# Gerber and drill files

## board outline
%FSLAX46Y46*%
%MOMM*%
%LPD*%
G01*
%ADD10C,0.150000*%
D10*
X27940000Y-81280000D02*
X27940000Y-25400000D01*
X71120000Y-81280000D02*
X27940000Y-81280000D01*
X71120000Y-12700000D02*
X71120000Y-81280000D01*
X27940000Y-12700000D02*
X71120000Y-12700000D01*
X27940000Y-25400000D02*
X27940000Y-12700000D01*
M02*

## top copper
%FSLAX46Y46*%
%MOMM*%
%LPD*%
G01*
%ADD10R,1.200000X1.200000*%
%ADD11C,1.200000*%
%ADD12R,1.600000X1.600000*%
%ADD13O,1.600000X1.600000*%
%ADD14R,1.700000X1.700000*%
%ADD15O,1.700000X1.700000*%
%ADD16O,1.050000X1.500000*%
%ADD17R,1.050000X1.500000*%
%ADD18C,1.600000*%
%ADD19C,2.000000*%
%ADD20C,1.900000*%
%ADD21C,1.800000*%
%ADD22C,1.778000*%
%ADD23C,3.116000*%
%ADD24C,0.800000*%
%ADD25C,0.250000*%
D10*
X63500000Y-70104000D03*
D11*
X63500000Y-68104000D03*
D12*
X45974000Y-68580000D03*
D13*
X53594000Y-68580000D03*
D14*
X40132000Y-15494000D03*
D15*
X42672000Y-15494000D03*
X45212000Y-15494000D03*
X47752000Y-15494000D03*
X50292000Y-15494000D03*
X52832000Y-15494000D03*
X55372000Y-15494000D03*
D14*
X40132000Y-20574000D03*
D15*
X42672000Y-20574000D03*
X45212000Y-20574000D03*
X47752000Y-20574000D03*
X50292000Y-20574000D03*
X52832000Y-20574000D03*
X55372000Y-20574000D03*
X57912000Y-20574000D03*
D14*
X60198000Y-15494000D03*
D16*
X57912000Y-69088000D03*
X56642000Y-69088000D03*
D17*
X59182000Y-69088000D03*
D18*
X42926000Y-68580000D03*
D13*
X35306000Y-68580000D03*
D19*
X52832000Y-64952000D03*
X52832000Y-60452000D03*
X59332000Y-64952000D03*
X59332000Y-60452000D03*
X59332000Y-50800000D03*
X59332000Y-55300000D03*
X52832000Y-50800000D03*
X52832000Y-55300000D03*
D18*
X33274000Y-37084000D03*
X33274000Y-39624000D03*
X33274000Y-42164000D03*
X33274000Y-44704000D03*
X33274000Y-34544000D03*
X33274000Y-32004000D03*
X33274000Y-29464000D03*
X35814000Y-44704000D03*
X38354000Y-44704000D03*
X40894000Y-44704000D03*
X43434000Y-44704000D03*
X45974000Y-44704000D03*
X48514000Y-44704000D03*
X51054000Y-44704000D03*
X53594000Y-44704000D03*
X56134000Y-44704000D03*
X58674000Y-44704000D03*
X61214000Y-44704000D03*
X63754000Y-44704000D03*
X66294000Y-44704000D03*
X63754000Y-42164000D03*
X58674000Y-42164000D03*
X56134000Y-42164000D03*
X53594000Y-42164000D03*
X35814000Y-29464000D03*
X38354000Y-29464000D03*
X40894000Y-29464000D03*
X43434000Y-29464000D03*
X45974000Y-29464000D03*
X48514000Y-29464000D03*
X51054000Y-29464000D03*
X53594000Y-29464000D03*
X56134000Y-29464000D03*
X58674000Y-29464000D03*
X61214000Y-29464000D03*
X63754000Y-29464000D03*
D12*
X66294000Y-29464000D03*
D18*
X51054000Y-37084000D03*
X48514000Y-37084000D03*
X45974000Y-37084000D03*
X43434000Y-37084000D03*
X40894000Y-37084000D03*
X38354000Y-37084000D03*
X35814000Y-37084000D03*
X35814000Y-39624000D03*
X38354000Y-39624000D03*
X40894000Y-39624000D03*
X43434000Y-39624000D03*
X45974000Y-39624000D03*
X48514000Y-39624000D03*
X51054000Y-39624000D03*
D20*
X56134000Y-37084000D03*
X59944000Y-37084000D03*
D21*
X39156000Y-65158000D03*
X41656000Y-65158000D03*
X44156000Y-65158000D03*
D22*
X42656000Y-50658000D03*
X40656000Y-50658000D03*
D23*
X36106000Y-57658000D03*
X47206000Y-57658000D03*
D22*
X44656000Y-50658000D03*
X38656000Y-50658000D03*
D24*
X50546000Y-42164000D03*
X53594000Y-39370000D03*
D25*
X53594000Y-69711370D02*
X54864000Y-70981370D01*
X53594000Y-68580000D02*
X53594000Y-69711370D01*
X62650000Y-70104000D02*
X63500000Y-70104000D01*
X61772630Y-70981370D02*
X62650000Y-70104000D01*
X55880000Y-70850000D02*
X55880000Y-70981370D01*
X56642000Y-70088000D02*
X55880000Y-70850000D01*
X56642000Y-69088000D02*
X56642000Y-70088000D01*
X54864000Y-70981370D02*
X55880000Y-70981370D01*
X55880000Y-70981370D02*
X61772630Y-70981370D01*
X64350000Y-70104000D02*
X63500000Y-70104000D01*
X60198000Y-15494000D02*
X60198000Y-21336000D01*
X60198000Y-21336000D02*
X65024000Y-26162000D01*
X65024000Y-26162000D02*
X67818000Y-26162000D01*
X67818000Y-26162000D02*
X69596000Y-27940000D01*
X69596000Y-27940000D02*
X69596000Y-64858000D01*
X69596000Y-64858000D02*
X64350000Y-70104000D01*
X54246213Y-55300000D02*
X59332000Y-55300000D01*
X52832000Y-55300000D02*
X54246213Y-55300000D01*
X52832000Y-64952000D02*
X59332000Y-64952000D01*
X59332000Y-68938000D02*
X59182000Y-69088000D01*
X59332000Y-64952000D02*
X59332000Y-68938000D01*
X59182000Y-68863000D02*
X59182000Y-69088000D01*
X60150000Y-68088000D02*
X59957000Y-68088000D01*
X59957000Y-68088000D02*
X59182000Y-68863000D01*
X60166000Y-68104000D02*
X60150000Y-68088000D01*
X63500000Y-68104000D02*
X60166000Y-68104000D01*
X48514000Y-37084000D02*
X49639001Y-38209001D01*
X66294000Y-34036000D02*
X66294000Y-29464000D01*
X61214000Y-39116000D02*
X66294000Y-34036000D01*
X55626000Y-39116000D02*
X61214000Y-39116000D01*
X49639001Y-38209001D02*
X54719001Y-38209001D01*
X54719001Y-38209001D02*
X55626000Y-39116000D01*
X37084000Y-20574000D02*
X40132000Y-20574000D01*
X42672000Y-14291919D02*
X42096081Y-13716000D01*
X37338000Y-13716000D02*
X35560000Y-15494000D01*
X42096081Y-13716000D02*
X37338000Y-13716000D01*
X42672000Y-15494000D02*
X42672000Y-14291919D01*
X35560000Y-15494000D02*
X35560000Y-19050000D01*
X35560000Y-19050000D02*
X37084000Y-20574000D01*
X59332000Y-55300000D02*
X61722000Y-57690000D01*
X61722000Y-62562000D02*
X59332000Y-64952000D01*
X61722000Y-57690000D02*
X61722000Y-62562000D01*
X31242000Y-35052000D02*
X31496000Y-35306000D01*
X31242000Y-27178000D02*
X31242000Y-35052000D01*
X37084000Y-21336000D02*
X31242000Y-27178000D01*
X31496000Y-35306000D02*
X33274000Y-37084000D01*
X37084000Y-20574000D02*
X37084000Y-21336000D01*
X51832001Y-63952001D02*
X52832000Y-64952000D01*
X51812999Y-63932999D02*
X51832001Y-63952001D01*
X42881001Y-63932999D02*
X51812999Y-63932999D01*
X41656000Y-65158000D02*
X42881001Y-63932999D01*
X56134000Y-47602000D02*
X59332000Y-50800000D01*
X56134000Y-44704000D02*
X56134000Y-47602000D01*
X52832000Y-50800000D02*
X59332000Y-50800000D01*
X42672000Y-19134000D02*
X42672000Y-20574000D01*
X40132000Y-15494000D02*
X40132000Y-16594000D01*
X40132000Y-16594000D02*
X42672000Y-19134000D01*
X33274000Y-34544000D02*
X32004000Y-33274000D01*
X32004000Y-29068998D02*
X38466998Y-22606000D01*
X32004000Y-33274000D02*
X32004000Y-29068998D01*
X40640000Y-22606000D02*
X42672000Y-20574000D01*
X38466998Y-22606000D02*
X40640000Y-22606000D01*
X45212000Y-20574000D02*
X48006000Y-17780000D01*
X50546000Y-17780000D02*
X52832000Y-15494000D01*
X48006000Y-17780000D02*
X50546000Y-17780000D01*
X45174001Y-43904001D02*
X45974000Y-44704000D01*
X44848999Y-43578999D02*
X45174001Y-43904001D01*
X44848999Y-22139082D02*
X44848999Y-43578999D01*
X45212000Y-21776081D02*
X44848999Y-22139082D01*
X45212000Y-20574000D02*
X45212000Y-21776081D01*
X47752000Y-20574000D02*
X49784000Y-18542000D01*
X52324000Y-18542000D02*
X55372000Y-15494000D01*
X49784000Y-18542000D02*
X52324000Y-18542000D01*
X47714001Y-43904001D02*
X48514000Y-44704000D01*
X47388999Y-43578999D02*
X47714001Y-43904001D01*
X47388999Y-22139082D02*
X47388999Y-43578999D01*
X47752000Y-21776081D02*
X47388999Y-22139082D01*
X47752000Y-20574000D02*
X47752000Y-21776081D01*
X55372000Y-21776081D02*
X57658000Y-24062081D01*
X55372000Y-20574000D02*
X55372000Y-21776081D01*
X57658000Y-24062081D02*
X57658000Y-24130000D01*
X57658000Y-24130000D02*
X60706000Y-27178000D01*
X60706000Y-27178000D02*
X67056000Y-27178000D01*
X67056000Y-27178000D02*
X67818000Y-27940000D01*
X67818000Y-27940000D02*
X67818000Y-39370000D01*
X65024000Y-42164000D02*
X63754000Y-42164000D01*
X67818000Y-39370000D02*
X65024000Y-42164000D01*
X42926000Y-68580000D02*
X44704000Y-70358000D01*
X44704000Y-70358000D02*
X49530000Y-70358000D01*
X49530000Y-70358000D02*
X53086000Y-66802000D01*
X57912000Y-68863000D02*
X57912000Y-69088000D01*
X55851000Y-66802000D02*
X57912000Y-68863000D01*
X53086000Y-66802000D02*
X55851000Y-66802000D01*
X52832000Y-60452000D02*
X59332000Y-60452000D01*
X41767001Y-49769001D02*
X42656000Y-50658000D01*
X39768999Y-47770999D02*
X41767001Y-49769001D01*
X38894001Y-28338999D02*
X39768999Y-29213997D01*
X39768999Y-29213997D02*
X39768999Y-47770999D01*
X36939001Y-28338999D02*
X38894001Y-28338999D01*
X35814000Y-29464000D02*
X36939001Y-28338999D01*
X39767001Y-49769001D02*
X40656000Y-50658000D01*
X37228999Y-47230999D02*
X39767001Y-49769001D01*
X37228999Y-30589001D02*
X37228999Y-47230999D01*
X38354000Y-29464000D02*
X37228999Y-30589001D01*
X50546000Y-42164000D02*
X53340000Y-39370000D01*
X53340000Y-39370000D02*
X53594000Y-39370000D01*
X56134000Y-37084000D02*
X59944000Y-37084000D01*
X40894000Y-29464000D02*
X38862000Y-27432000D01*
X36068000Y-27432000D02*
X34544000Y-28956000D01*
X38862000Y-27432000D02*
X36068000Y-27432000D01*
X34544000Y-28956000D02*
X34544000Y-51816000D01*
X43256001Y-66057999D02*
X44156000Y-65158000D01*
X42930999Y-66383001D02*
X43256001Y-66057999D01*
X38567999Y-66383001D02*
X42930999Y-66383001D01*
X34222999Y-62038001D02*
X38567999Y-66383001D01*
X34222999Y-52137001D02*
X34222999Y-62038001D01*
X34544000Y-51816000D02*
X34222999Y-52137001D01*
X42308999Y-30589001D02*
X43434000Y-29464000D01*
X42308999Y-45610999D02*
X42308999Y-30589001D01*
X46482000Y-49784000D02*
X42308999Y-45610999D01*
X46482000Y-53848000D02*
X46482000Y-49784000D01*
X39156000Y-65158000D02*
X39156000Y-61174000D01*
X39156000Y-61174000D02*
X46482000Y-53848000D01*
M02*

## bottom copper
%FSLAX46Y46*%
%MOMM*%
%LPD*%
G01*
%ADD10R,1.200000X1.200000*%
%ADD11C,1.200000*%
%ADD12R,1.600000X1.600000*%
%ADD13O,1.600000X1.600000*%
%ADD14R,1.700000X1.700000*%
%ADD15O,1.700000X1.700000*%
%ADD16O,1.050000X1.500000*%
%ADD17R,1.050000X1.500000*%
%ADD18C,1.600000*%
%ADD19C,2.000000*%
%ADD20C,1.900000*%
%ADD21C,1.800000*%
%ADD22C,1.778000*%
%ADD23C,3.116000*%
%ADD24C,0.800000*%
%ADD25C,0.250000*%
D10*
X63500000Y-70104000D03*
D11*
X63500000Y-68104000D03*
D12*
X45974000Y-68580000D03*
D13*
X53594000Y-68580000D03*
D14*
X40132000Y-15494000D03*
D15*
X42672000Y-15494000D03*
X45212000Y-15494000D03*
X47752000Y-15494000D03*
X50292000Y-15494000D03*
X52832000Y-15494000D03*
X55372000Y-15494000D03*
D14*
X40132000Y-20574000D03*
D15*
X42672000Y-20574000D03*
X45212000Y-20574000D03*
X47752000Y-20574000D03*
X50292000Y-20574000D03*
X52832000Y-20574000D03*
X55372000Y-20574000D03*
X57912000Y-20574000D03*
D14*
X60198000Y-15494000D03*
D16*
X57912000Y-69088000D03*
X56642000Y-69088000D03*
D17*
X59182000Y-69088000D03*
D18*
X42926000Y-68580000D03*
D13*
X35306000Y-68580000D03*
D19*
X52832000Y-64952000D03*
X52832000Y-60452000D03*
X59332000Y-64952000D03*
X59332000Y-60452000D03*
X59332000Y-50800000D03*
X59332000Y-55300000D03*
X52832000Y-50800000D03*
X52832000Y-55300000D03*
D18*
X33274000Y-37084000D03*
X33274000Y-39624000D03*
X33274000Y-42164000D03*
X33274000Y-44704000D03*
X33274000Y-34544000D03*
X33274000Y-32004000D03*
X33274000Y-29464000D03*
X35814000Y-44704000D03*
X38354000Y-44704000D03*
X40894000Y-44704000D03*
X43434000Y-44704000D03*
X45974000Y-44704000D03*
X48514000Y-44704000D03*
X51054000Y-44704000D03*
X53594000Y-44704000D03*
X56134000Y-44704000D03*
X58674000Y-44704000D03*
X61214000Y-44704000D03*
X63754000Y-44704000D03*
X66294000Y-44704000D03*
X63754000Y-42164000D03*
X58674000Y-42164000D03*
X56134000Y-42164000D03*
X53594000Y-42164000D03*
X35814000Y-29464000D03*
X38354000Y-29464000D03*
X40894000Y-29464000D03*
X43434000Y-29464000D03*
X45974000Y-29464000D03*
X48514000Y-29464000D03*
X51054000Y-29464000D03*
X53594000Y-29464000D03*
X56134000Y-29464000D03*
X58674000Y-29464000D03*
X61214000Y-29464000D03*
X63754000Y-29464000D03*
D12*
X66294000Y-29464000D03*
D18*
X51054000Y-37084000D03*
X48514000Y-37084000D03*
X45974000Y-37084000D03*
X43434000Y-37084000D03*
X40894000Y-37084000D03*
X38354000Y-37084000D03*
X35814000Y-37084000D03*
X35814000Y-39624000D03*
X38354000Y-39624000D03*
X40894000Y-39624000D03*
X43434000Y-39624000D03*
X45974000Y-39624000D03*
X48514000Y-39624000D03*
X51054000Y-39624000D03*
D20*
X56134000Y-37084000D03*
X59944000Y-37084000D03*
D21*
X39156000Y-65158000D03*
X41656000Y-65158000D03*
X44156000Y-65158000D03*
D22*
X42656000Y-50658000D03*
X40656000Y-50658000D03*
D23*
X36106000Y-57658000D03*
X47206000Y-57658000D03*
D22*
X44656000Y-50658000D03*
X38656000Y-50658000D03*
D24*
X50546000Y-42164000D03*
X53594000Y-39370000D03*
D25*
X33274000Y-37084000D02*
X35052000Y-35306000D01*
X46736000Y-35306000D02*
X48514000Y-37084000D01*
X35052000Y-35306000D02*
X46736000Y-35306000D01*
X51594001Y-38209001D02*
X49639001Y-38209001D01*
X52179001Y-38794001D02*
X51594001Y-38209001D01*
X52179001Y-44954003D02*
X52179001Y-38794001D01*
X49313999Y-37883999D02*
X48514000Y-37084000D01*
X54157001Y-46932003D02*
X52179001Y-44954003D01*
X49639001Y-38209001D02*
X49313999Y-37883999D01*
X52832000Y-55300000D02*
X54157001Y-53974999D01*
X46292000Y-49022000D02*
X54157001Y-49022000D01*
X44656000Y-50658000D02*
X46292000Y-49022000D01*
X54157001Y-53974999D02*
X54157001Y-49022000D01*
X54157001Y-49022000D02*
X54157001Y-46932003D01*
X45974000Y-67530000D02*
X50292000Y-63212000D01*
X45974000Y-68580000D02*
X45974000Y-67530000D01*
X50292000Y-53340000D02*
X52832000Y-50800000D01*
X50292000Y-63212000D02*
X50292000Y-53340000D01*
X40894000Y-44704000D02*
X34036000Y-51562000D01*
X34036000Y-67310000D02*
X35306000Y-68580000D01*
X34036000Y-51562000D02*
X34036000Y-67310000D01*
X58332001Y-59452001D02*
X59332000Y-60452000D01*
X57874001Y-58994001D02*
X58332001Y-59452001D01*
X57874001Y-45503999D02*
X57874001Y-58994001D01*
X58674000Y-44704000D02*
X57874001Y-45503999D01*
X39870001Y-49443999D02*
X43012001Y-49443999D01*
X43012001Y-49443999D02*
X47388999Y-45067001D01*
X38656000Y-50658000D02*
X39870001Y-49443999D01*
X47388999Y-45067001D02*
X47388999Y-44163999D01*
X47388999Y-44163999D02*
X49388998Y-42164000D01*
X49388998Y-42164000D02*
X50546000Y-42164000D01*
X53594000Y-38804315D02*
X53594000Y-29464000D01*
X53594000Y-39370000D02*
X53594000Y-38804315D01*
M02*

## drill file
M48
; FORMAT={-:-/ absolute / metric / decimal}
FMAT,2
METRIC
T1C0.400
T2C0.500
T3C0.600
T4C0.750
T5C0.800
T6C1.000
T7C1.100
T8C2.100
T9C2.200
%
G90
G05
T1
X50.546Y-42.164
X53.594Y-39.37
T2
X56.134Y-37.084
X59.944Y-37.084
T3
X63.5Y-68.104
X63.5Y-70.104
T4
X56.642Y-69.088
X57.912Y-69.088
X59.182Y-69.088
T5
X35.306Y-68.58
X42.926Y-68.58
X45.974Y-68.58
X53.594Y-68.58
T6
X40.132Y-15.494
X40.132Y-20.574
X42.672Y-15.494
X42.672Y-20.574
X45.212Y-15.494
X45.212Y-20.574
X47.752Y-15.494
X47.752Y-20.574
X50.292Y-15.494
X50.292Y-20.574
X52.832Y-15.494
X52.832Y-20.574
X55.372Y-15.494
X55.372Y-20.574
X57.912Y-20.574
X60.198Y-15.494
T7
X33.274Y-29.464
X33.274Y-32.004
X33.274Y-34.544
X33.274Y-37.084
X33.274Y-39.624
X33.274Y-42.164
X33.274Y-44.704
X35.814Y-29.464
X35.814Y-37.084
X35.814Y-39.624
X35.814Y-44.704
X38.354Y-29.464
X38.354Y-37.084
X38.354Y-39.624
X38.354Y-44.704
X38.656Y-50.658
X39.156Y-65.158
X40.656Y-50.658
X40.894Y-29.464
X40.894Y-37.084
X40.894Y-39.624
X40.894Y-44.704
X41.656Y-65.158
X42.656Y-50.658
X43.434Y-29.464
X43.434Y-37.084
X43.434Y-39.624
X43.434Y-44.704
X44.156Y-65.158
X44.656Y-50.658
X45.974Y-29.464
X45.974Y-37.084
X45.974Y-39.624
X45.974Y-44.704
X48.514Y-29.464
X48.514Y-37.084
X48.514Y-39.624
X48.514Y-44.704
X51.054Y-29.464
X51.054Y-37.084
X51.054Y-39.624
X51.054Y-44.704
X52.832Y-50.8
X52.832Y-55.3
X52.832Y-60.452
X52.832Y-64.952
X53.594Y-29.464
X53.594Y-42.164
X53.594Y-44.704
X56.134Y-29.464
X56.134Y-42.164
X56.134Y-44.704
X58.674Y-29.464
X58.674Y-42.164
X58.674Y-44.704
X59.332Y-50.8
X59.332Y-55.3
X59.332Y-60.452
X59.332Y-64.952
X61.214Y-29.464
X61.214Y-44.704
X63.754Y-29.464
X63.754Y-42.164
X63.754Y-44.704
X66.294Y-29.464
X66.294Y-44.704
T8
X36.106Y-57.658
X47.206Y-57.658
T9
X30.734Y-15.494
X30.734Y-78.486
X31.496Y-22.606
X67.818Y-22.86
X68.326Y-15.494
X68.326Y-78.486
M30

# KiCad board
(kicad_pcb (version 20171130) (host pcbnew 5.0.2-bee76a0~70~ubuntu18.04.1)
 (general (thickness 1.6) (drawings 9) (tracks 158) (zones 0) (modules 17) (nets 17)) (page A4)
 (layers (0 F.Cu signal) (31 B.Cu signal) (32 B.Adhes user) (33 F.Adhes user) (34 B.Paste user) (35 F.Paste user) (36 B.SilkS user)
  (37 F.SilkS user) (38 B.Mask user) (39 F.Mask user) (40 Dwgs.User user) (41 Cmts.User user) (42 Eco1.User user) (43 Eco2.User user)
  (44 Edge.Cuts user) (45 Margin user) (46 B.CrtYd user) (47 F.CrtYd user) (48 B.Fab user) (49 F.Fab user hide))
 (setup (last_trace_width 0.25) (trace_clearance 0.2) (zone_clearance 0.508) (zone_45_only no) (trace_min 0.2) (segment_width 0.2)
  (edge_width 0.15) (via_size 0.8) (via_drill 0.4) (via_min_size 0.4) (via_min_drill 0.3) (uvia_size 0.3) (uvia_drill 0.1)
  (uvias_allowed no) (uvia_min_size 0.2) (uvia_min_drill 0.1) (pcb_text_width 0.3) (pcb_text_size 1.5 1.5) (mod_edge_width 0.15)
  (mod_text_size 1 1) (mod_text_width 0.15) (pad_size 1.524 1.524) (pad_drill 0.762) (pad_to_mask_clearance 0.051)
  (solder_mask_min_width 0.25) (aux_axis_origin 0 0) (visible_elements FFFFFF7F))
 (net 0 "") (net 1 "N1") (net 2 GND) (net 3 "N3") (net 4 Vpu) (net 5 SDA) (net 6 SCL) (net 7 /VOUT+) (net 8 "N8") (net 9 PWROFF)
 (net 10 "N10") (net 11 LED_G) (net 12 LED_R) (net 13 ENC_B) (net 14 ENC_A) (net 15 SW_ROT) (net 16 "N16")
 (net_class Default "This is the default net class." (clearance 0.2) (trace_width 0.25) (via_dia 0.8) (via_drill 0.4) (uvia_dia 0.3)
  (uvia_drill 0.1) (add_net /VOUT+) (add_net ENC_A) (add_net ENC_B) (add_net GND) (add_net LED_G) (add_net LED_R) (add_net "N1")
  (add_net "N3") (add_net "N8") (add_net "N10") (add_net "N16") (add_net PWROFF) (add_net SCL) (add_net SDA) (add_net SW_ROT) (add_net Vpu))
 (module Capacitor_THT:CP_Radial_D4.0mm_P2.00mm (layer F.Cu) (at 63.5 70.104 90)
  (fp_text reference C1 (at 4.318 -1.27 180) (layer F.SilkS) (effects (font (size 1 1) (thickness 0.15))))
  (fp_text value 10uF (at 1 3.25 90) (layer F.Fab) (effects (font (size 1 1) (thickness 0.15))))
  (pad 1 thru_hole rect (at 0 0 90) (size 1.2 1.2) (drill 0.6) (layers *.Cu *.Mask) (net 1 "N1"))
  (pad 2 thru_hole circle (at 2 0 90) (size 1.2 1.2) (drill 0.6) (layers *.Cu *.Mask) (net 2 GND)))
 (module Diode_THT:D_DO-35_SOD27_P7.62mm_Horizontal (layer F.Cu) (at 45.974 68.58)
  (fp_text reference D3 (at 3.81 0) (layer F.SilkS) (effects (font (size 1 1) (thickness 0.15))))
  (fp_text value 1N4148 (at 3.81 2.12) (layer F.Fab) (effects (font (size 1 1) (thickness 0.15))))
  (pad 1 thru_hole rect (at 0 0) (size 1.6 1.6) (drill 0.8) (layers *.Cu *.Mask) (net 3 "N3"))
  (pad 2 thru_hole oval (at 7.62 0) (size 1.6 1.6) (drill 0.8) (layers *.Cu *.Mask) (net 1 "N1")))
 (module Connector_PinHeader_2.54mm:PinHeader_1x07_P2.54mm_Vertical (layer F.Cu) (at 40.132 15.494 90)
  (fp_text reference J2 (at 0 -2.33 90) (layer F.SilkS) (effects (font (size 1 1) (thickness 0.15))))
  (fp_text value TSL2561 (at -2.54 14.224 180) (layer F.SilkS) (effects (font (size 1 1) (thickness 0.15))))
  (pad 1 thru_hole rect (at 0 0 90) (size 1.7 1.7) (drill 1) (layers *.Cu *.Mask) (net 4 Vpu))
  (pad 2 thru_hole oval (at 0 2.54 90) (size 1.7 1.7) (drill 1) (layers *.Cu *.Mask) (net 2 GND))
  (pad 3 thru_hole oval (at 0 5.08 90) (size 1.7 1.7) (drill 1) (layers *.Cu *.Mask))
  (pad 4 thru_hole oval (at 0 7.62 90) (size 1.7 1.7) (drill 1) (layers *.Cu *.Mask))
  (pad 5 thru_hole oval (at 0 10.16 90) (size 1.7 1.7) (drill 1) (layers *.Cu *.Mask))
  (pad 6 thru_hole oval (at 0 12.7 90) (size 1.7 1.7) (drill 1) (layers *.Cu *.Mask) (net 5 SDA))
  (pad 7 thru_hole oval (at 0 15.24 90) (size 1.7 1.7) (drill 1) (layers *.Cu *.Mask) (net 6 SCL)))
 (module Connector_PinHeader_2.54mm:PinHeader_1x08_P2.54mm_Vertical (layer F.Cu) (at 40.132 20.574 90)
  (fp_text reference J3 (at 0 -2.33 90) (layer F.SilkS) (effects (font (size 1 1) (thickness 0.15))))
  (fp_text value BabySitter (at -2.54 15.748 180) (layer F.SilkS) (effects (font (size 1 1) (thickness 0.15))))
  (pad 1 thru_hole rect (at 0 0 90) (size 1.7 1.7) (drill 1) (layers *.Cu *.Mask) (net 2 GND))
  (pad 2 thru_hole oval (at 0 2.54 90) (size 1.7 1.7) (drill 1) (layers *.Cu *.Mask) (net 4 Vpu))
  (pad 3 thru_hole oval (at 0 5.08 90) (size 1.7 1.7) (drill 1) (layers *.Cu *.Mask) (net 5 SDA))
  (pad 4 thru_hole oval (at 0 7.62 90) (size 1.7 1.7) (drill 1) (layers *.Cu *.Mask) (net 6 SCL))
  (pad 5 thru_hole oval (at 0 10.16 90) (size 1.7 1.7) (drill 1) (layers *.Cu *.Mask))
  (pad 6 thru_hole oval (at 0 12.7 90) (size 1.7 1.7) (drill 1) (layers *.Cu *.Mask))
  (pad 7 thru_hole oval (at 0 15.24 90) (size 1.7 1.7) (drill 1) (layers *.Cu *.Mask) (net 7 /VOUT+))
  (pad 8 thru_hole oval (at 0 17.78 90) (size 1.7 1.7) (drill 1) (layers *.Cu *.Mask)))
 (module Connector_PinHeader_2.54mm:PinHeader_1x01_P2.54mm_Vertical (layer F.Cu) (at 60.198 15.494)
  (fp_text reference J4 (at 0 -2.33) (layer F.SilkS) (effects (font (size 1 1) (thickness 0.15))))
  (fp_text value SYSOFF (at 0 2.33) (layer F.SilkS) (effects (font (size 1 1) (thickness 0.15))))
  (pad 1 thru_hole rect (at 0 0) (size 1.7 1.7) (drill 1) (layers *.Cu *.Mask) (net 1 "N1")))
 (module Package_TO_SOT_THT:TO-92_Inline (layer F.Cu) (at 59.182 69.088 180)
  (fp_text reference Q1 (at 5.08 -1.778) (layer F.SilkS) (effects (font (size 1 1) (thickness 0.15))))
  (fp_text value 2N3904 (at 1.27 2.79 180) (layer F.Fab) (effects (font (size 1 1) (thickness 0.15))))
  (pad 2 thru_hole oval (at 1.27 0 180) (size 1.05 1.5) (drill 0.75) (layers *.Cu *.Mask) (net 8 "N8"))
  (pad 3 thru_hole oval (at 2.54 0 180) (size 1.05 1.5) (drill 0.75) (layers *.Cu *.Mask) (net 1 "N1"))
  (pad 1 thru_hole rect (at 0 0 180) (size 1.05 1.5) (drill 0.75) (layers *.Cu *.Mask) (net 2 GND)))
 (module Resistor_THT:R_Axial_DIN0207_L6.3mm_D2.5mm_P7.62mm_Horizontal (layer F.Cu) (at 42.926 68.58 180)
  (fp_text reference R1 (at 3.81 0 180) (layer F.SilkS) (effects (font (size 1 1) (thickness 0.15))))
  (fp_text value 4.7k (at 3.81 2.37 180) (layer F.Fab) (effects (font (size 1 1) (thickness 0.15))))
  (pad 1 thru_hole circle (at 0 0 180) (size 1.6 1.6) (drill 0.8) (layers *.Cu *.Mask) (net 8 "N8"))
  (pad 2 thru_hole oval (at 7.62 0 180) (size 1.6 1.6) (drill 0.8) (layers *.Cu *.Mask) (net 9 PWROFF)))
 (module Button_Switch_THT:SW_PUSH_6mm (layer F.Cu) (at 52.832 60.452)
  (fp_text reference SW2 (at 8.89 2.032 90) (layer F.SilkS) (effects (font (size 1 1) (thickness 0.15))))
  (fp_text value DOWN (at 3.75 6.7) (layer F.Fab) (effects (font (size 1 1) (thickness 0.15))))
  (pad 2 thru_hole circle (at 0 4.5 90) (size 2 2) (drill 1.1) (layers *.Cu *.Mask) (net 2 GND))
  (pad 1 thru_hole circle (at 0 0 90) (size 2 2) (drill 1.1) (layers *.Cu *.Mask) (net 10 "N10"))
  (pad 2 thru_hole circle (at 6.5 4.5 90) (size 2 2) (drill 1.1) (layers *.Cu *.Mask) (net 2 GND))
  (pad 1 thru_hole circle (at 6.5 0 90) (size 2 2) (drill 1.1) (layers *.Cu *.Mask) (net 10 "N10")))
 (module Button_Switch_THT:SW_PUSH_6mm (layer F.Cu) (at 52.832 50.8)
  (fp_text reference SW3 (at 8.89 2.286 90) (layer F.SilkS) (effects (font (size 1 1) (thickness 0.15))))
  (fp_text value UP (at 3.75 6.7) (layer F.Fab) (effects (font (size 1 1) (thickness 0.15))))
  (pad 1 thru_hole circle (at 6.5 0 90) (size 2 2) (drill 1.1) (layers *.Cu *.Mask) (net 3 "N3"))
  (pad 2 thru_hole circle (at 6.5 4.5 90) (size 2 2) (drill 1.1) (layers *.Cu *.Mask) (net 2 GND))
  (pad 1 thru_hole circle (at 0 0 90) (size 2 2) (drill 1.1) (layers *.Cu *.Mask) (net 3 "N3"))
  (pad 2 thru_hole circle (at 0 4.5 90) (size 2 2) (drill 1.1) (layers *.Cu *.Mask) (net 2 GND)))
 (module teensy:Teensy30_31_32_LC (layer F.Cu) (at 49.784 37.084 180)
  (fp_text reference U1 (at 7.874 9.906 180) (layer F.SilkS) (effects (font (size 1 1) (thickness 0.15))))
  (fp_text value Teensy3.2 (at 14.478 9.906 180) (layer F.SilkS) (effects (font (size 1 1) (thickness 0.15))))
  (pad 17 thru_hole circle (at 16.51 0 180) (size 1.6 1.6) (drill 1.1) (layers *.Cu *.Mask F.SilkS) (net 2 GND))
  (pad 18 thru_hole circle (at 16.51 -2.54 180) (size 1.6 1.6) (drill 1.1) (layers *.Cu *.Mask F.SilkS))
  (pad 19 thru_hole circle (at 16.51 -5.08 180) (size 1.6 1.6) (drill 1.1) (layers *.Cu *.Mask F.SilkS))
  (pad 20 thru_hole circle (at 16.51 -7.62 180) (size 1.6 1.6) (drill 1.1) (layers *.Cu *.Mask F.SilkS))
  (pad 16 thru_hole circle (at 16.51 2.54 180) (size 1.6 1.6) (drill 1.1) (layers *.Cu *.Mask F.SilkS) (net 4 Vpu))
  (pad 15 thru_hole circle (at 16.51 5.08 180) (size 1.6 1.6) (drill 1.1) (layers *.Cu *.Mask F.SilkS))
  (pad 14 thru_hole circle (at 16.51 7.62 180) (size 1.6 1.6) (drill 1.1) (layers *.Cu *.Mask F.SilkS))
  (pad 21 thru_hole circle (at 13.97 -7.62 180) (size 1.6 1.6) (drill 1.1) (layers *.Cu *.Mask F.SilkS))
  (pad 22 thru_hole circle (at 11.43 -7.62 180) (size 1.6 1.6) (drill 1.1) (layers *.Cu *.Mask F.SilkS))
  (pad 23 thru_hole circle (at 8.89 -7.62 180) (size 1.6 1.6) (drill 1.1) (layers *.Cu *.Mask F.SilkS) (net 9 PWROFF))
  (pad 24 thru_hole circle (at 6.35 -7.62 180) (size 1.6 1.6) (drill 1.1) (layers *.Cu *.Mask F.SilkS))
  (pad 25 thru_hole circle (at 3.81 -7.62 180) (size 1.6 1.6) (drill 1.1) (layers *.Cu *.Mask F.SilkS) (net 5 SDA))
  (pad 26 thru_hole circle (at 1.27 -7.62 180) (size 1.6 1.6) (drill 1.1) (layers *.Cu *.Mask F.SilkS) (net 6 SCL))
  (pad 27 thru_hole circle (at -1.27 -7.62 180) (size 1.6 1.6) (drill 1.1) (layers *.Cu *.Mask F.SilkS))
  (pad 28 thru_hole circle (at -3.81 -7.62 180) (size 1.6 1.6) (drill 1.1) (layers *.Cu *.Mask F.SilkS))
  (pad 29 thru_hole circle (at -6.35 -7.62 180) (size 1.6 1.6) (drill 1.1) (layers *.Cu *.Mask F.SilkS) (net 3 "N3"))
  (pad 30 thru_hole circle (at -8.89 -7.62 180) (size 1.6 1.6) (drill 1.1) (layers *.Cu *.Mask F.SilkS) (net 10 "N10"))
  (pad 31 thru_hole circle (at -11.43 -7.62 180) (size 1.6 1.6) (drill 1.1) (layers *.Cu *.Mask F.SilkS))
  (pad 32 thru_hole circle (at -13.97 -7.62 180) (size 1.6 1.6) (drill 1.1) (layers *.Cu *.Mask F.SilkS))
  (pad 33 thru_hole circle (at -16.51 -7.62 180) (size 1.6 1.6) (drill 1.1) (layers *.Cu *.Mask F.SilkS))
  (pad 34 thru_hole circle (at -13.97 -5.08 180) (size 1.6 1.6) (drill 1.1) (layers *.Cu *.Mask F.SilkS) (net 7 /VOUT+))
  (pad 35 thru_hole circle (at -8.89 -5.08 180) (size 1.6 1.6) (drill 1.1) (layers *.Cu *.Mask F.SilkS))
  (pad 36 thru_hole circle (at -6.35 -5.08 180) (size 1.6 1.6) (drill 1.1) (layers *.Cu *.Mask F.SilkS))
  (pad 37 thru_hole circle (at -3.81 -5.08 180) (size 1.6 1.6) (drill 1.1) (layers *.Cu *.Mask F.SilkS))
  (pad 13 thru_hole circle (at 13.97 7.62 180) (size 1.6 1.6) (drill 1.1) (layers *.Cu *.Mask F.SilkS) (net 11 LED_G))
  (pad 12 thru_hole circle (at 11.43 7.62 180) (size 1.6 1.6) (drill 1.1) (layers *.Cu *.Mask F.SilkS) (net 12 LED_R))
  (pad 11 thru_hole circle (at 8.89 7.62 180) (size 1.6 1.6) (drill 1.1) (layers *.Cu *.Mask F.SilkS) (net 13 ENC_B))
  (pad 10 thru_hole circle (at 6.35 7.62 180) (size 1.6 1.6) (drill 1.1) (layers *.Cu *.Mask F.SilkS) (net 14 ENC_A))
  (pad 9 thru_hole circle (at 3.81 7.62 180) (size 1.6 1.6) (drill 1.1) (layers *.Cu *.Mask F.SilkS))
  (pad 8 thru_hole circle (at 1.27 7.62 180) (size 1.6 1.6) (drill 1.1) (layers *.Cu *.Mask F.SilkS))
  (pad 7 thru_hole circle (at -1.27 7.62 180) (size 1.6 1.6) (drill 1.1) (layers *.Cu *.Mask F.SilkS))
  (pad 6 thru_hole circle (at -3.81 7.62 180) (size 1.6 1.6) (drill 1.1) (layers *.Cu *.Mask F.SilkS) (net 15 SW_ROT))
  (pad 5 thru_hole circle (at -6.35 7.62 180) (size 1.6 1.6) (drill 1.1) (layers *.Cu *.Mask F.SilkS))
  (pad 4 thru_hole circle (at -8.89 7.62 180) (size 1.6 1.6) (drill 1.1) (layers *.Cu *.Mask F.SilkS))
  (pad 3 thru_hole circle (at -11.43 7.62 180) (size 1.6 1.6) (drill 1.1) (layers *.Cu *.Mask F.SilkS))
  (pad 2 thru_hole circle (at -13.97 7.62 180) (size 1.6 1.6) (drill 1.1) (layers *.Cu *.Mask F.SilkS))
  (pad 1 thru_hole rect (at -16.51 7.62 180) (size 1.6 1.6) (drill 1.1) (layers *.Cu *.Mask F.SilkS) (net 2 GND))
  (pad 38 thru_hole circle (at -1.27 0 180) (size 1.6 1.6) (drill 1.1) (layers *.Cu *.Mask))
  (pad 39 thru_hole circle (at 1.27 0 180) (size 1.6 1.6) (drill 1.1) (layers *.Cu *.Mask) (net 2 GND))
  (pad 40 thru_hole circle (at 3.81 0 180) (size 1.6 1.6) (drill 1.1) (layers *.Cu *.Mask))
  (pad 41 thru_hole circle (at 6.35 0 180) (size 1.6 1.6) (drill 1.1) (layers *.Cu *.Mask))
  (pad 42 thru_hole circle (at 8.89 0 180) (size 1.6 1.6) (drill 1.1) (layers *.Cu *.Mask))
  (pad 43 thru_hole circle (at 11.43 0 180) (size 1.6 1.6) (drill 1.1) (layers *.Cu *.Mask))
  (pad 44 thru_hole circle (at 13.97 0 180) (size 1.6 1.6) (drill 1.1) (layers *.Cu *.Mask))
  (pad 45 thru_hole circle (at 13.97 -2.54 180) (size 1.6 1.6) (drill 1.1) (layers *.Cu *.Mask))
  (pad 46 thru_hole circle (at 11.43 -2.54 180) (size 1.6 1.6) (drill 1.1) (layers *.Cu *.Mask))
  (pad 47 thru_hole circle (at 8.89 -2.54 180) (size 1.6 1.6) (drill 1.1) (layers *.Cu *.Mask))
  (pad 48 thru_hole circle (at 6.35 -2.54 180) (size 1.6 1.6) (drill 1.1) (layers *.Cu *.Mask))
  (pad 49 thru_hole circle (at 3.81 -2.54 180) (size 1.6 1.6) (drill 1.1) (layers *.Cu *.Mask))
  (pad 50 thru_hole circle (at 1.27 -2.54 180) (size 1.6 1.6) (drill 1.1) (layers *.Cu *.Mask))
  (pad 51 thru_hole circle (at -1.27 -2.54 180) (size 1.6 1.6) (drill 1.1) (layers *.Cu *.Mask))
  (pad 52 thru_hole circle (at -6.35 0 180) (size 1.9 1.9) (drill 0.5) (layers *.Cu *.Mask F.SilkS) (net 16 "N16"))
  (pad 52 thru_hole circle (at -10.16 0 180) (size 1.9 1.9) (drill 0.5) (layers *.Cu *.Mask F.SilkS) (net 16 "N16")))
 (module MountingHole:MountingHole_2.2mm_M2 (layer F.Cu) (at 30.734 15.494)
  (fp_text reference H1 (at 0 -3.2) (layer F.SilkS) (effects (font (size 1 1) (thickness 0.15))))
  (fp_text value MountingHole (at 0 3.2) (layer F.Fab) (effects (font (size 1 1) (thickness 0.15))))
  (pad 1 np_thru_hole circle (at 0 0) (size 2.2 2.2) (drill 2.2) (layers *.Cu *.Mask)))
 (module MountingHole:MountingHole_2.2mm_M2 (layer F.Cu) (at 68.326 78.486)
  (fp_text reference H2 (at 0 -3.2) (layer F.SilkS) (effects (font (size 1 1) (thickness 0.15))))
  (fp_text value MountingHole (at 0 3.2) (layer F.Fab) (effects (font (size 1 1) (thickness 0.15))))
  (pad 1 np_thru_hole circle (at 0 0) (size 2.2 2.2) (drill 2.2) (layers *.Cu *.Mask)))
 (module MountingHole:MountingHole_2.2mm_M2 (layer F.Cu) (at 68.326 15.494)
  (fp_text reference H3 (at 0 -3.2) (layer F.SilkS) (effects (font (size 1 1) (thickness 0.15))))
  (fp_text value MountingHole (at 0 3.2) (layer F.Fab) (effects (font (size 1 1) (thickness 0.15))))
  (pad 1 np_thru_hole circle (at 0 0) (size 2.2 2.2) (drill 2.2) (layers *.Cu *.Mask)))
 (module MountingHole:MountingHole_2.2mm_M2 (layer F.Cu) (at 67.818 22.86)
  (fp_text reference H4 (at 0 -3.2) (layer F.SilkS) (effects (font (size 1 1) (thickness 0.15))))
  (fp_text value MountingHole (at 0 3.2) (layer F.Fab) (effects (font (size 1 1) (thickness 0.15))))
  (pad 1 np_thru_hole circle (at 0 0) (size 2.2 2.2) (drill 2.2) (layers *.Cu *.Mask)))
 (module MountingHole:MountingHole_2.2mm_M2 (layer F.Cu) (at 30.734 78.486)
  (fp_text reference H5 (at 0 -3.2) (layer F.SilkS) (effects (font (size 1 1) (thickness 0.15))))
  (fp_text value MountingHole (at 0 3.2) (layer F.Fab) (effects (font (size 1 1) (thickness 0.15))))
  (pad 1 np_thru_hole circle (at 0 0) (size 2.2 2.2) (drill 2.2) (layers *.Cu *.Mask)))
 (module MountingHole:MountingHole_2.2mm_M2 (layer F.Cu) (at 31.496 22.606)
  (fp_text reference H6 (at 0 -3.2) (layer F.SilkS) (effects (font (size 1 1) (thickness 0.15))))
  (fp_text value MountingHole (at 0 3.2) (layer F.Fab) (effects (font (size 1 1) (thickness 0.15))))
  (pad 1 np_thru_hole circle (at 0 0) (size 2.2 2.2) (drill 2.2) (layers *.Cu *.Mask)))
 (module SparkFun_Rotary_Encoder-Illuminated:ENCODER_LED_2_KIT (layer F.Cu) (at 41.656 57.658)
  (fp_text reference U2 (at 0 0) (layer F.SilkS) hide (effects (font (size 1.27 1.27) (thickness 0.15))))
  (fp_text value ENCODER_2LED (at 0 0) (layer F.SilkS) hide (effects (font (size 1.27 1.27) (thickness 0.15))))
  (pad A thru_hole circle (at -2.5 7.5) (size 1.8 1.8) (drill 1.1) (layers *.Cu *.Mask) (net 14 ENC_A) (solder_mask_margin 0.1016))
  (pad C thru_hole circle (at 0 7.5) (size 1.8 1.8) (drill 1.1) (layers *.Cu *.Mask) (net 2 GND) (solder_mask_margin 0.1016))
  (pad B thru_hole circle (at 2.5 7.5) (size 1.8 1.8) (drill 1.1) (layers *.Cu *.Mask) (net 13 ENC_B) (solder_mask_margin 0.1016))
  (pad +G thru_hole circle (at 1 -7) (size 1.778 1.778) (drill 1.1) (layers *.Cu *.Mask) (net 11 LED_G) (solder_mask_margin 0.1016))
  (pad +R thru_hole circle (at -1 -7) (size 1.778 1.778) (drill 1.1) (layers *.Cu *.Mask) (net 12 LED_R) (solder_mask_margin 0.1016))
  (pad P$1 thru_hole circle (at -5.55 0) (size 3.116 3.116) (drill 2.1) (layers *.Cu *.Mask) (solder_mask_margin 0.1016))
  (pad P$2 thru_hole circle (at 5.55 0) (size 3.116 3.116) (drill 2.1) (layers *.Cu *.Mask) (solder_mask_margin 0.1016))
  (pad GND thru_hole circle (at 3 -7) (size 1.778 1.778) (drill 1.1) (layers *.Cu *.Mask) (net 2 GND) (solder_mask_margin 0.1016))
  (pad SW thru_hole circle (at -3 -7) (size 1.778 1.778) (drill 1.1) (layers *.Cu *.Mask) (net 15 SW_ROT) (solder_mask_margin 0.1016)))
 (gr_line (start 27.94 81.28) (end 27.94 25.4) (layer Edge.Cuts) (width 0.15))
 (gr_line (start 71.12 81.28) (end 27.94 81.28) (layer Edge.Cuts) (width 0.15))
 (gr_line (start 71.12 12.7) (end 71.12 81.28) (layer Edge.Cuts) (width 0.15))
 (gr_line (start 27.94 12.7) (end 71.12 12.7) (layer Edge.Cuts) (width 0.15))
 (gr_line (start 27.94 25.4) (end 27.94 12.7) (layer Edge.Cuts) (width 0.15))
 (segment (start 53.594 69.71137) (end 54.864 70.98137) (width 0.25) (layer F.Cu) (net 1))
 (segment (start 53.594 68.58) (end 53.594 69.71137) (width 0.25) (layer F.Cu) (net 1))
 (segment (start 62.65 70.104) (end 63.5 70.104) (width 0.25) (layer F.Cu) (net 1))
 (segment (start 61.77263 70.98137) (end 62.65 70.104) (width 0.25) (layer F.Cu) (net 1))
 (segment (start 55.88 70.85) (end 55.88 70.98137) (width 0.25) (layer F.Cu) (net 1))
 (segment (start 56.642 70.088) (end 55.88 70.85) (width 0.25) (layer F.Cu) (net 1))
 (segment (start 56.642 69.088) (end 56.642 70.088) (width 0.25) (layer F.Cu) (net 1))
 (segment (start 54.864 70.98137) (end 55.88 70.98137) (width 0.25) (layer F.Cu) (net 1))
 (segment (start 55.88 70.98137) (end 61.77263 70.98137) (width 0.25) (layer F.Cu) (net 1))
 (segment (start 64.35 70.104) (end 63.5 70.104) (width 0.25) (layer F.Cu) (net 1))
 (segment (start 60.198 15.494) (end 60.198 21.336) (width 0.25) (layer F.Cu) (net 1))
 (segment (start 60.198 21.336) (end 65.024 26.162) (width 0.25) (layer F.Cu) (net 1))
 (segment (start 65.024 26.162) (end 67.818 26.162) (width 0.25) (layer F.Cu) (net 1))
 (segment (start 67.818 26.162) (end 69.596 27.94) (width 0.25) (layer F.Cu) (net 1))
 (segment (start 69.596 27.94) (end 69.596 64.858) (width 0.25) (layer F.Cu) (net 1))
 (segment (start 69.596 64.858) (end 64.35 70.104) (width 0.25) (layer F.Cu) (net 1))
 (segment (start 54.246213 55.3) (end 59.332 55.3) (width 0.25) (layer F.Cu) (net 2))
 (segment (start 52.832 55.3) (end 54.246213 55.3) (width 0.25) (layer F.Cu) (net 2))
 (segment (start 52.832 64.952) (end 59.332 64.952) (width 0.25) (layer F.Cu) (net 2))
 (segment (start 59.332 68.938) (end 59.182 69.088) (width 0.25) (layer F.Cu) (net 2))
 (segment (start 59.332 64.952) (end 59.332 68.938) (width 0.25) (layer F.Cu) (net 2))
 (segment (start 59.182 68.863) (end 59.182 69.088) (width 0.25) (layer F.Cu) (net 2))
 (segment (start 60.15 68.088) (end 59.957 68.088) (width 0.25) (layer F.Cu) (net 2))
 (segment (start 59.957 68.088) (end 59.182 68.863) (width 0.25) (layer F.Cu) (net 2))
 (segment (start 60.166 68.104) (end 60.15 68.088) (width 0.25) (layer F.Cu) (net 2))
 (segment (start 63.5 68.104) (end 60.166 68.104) (width 0.25) (layer F.Cu) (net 2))
 (segment (start 48.514 37.084) (end 49.639001 38.209001) (width 0.25) (layer F.Cu) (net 2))
 (segment (start 66.294 34.036) (end 66.294 29.464) (width 0.25) (layer F.Cu) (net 2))
 (segment (start 61.214 39.116) (end 66.294 34.036) (width 0.25) (layer F.Cu) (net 2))
 (segment (start 55.626 39.116) (end 61.214 39.116) (width 0.25) (layer F.Cu) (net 2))
 (segment (start 49.639001 38.209001) (end 54.719001 38.209001) (width 0.25) (layer F.Cu) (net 2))
 (segment (start 54.719001 38.209001) (end 55.626 39.116) (width 0.25) (layer F.Cu) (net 2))
 (segment (start 37.084 20.574) (end 40.132 20.574) (width 0.25) (layer F.Cu) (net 2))
 (segment (start 42.672 14.291919) (end 42.096081 13.716) (width 0.25) (layer F.Cu) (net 2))
 (segment (start 37.338 13.716) (end 35.56 15.494) (width 0.25) (layer F.Cu) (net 2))
 (segment (start 42.096081 13.716) (end 37.338 13.716) (width 0.25) (layer F.Cu) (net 2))
 (segment (start 42.672 15.494) (end 42.672 14.291919) (width 0.25) (layer F.Cu) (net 2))
 (segment (start 35.56 15.494) (end 35.56 19.05) (width 0.25) (layer F.Cu) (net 2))
 (segment (start 35.56 19.05) (end 37.084 20.574) (width 0.25) (layer F.Cu) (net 2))
 (segment (start 33.274 37.084) (end 35.052 35.306) (width 0.25) (layer B.Cu) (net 2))
 (segment (start 46.736 35.306) (end 48.514 37.084) (width 0.25) (layer B.Cu) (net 2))
 (segment (start 35.052 35.306) (end 46.736 35.306) (width 0.25) (layer B.Cu) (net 2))
 (segment (start 59.332 55.3) (end 61.722 57.69) (width 0.25) (layer F.Cu) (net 2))
 (segment (start 61.722 62.562) (end 59.332 64.952) (width 0.25) (layer F.Cu) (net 2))
 (segment (start 61.722 57.69) (end 61.722 62.562) (width 0.25) (layer F.Cu) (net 2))
 (segment (start 31.242 35.052) (end 31.496 35.306) (width 0.25) (layer F.Cu) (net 2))
 (segment (start 31.242 27.178) (end 31.242 35.052) (width 0.25) (layer F.Cu) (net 2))
 (segment (start 37.084 21.336) (end 31.242 27.178) (width 0.25) (layer F.Cu) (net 2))
 (segment (start 31.496 35.306) (end 33.274 37.084) (width 0.25) (layer F.Cu) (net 2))
 (segment (start 37.084 20.574) (end 37.084 21.336) (width 0.25) (layer F.Cu) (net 2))
 (segment (start 51.594001 38.209001) (end 49.639001 38.209001) (width 0.25) (layer B.Cu) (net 2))
 (segment (start 52.179001 38.794001) (end 51.594001 38.209001) (width 0.25) (layer B.Cu) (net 2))
 (segment (start 52.179001 44.954003) (end 52.179001 38.794001) (width 0.25) (layer B.Cu) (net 2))
 (segment (start 49.313999 37.883999) (end 48.514 37.084) (width 0.25) (layer B.Cu) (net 2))
 (segment (start 54.157001 46.932003) (end 52.179001 44.954003) (width 0.25) (layer B.Cu) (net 2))
 (segment (start 49.639001 38.209001) (end 49.313999 37.883999) (width 0.25) (layer B.Cu) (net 2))
 (segment (start 52.832 55.3) (end 54.157001 53.974999) (width 0.25) (layer B.Cu) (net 2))
 (segment (start 46.292 49.022) (end 54.157001 49.022) (width 0.25) (layer B.Cu) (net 2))
 (segment (start 44.656 50.658) (end 46.292 49.022) (width 0.25) (layer B.Cu) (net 2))
 (segment (start 54.157001 53.974999) (end 54.157001 49.022) (width 0.25) (layer B.Cu) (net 2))
 (segment (start 54.157001 49.022) (end 54.157001 46.932003) (width 0.25) (layer B.Cu) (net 2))
 (segment (start 51.832001 63.952001) (end 52.832 64.952) (width 0.25) (layer F.Cu) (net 2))
 (segment (start 51.812999 63.932999) (end 51.832001 63.952001) (width 0.25) (layer F.Cu) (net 2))
 (segment (start 42.881001 63.932999) (end 51.812999 63.932999) (width 0.25) (layer F.Cu) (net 2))
 (segment (start 41.656 65.158) (end 42.881001 63.932999) (width 0.25) (layer F.Cu) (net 2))
 (segment (start 56.134 47.602) (end 59.332 50.8) (width 0.25) (layer F.Cu) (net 3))
 (segment (start 56.134 44.704) (end 56.134 47.602) (width 0.25) (layer F.Cu) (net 3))
 (segment (start 52.832 50.8) (end 59.332 50.8) (width 0.25) (layer F.Cu) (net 3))
 (segment (start 45.974 67.53) (end 50.292 63.212) (width 0.25) (layer B.Cu) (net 3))
 (segment (start 45.974 68.58) (end 45.974 67.53) (width 0.25) (layer B.Cu) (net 3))
 (segment (start 50.292 53.34) (end 52.832 50.8) (width 0.25) (layer B.Cu) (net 3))
 (segment (start 50.292 63.212) (end 50.292 53.34) (width 0.25) (layer B.Cu) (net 3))
 (segment (start 42.672 19.134) (end 42.672 20.574) (width 0.25) (layer F.Cu) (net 4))
 (segment (start 40.132 15.494) (end 40.132 16.594) (width 0.25) (layer F.Cu) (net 4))
 (segment (start 40.132 16.594) (end 42.672 19.134) (width 0.25) (layer F.Cu) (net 4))
 (segment (start 33.274 34.544) (end 32.004 33.274) (width 0.25) (layer F.Cu) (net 4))
 (segment (start 32.004 29.068998) (end 38.466998 22.606) (width 0.25) (layer F.Cu) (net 4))
 (segment (start 32.004 33.274) (end 32.004 29.068998) (width 0.25) (layer F.Cu) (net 4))
 (segment (start 40.64 22.606) (end 42.672 20.574) (width 0.25) (layer F.Cu) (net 4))
 (segment (start 38.466998 22.606) (end 40.64 22.606) (width 0.25) (layer F.Cu) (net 4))
 (segment (start 45.212 20.574) (end 48.006 17.78) (width 0.25) (layer F.Cu) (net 5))
 (segment (start 50.546 17.78) (end 52.832 15.494) (width 0.25) (layer F.Cu) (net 5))
 (segment (start 48.006 17.78) (end 50.546 17.78) (width 0.25) (layer F.Cu) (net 5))
 (segment (start 45.174001 43.904001) (end 45.974 44.704) (width 0.25) (layer F.Cu) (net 5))
 (segment (start 44.848999 43.578999) (end 45.174001 43.904001) (width 0.25) (layer F.Cu) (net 5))
 (segment (start 44.848999 22.139082) (end 44.848999 43.578999) (width 0.25) (layer F.Cu) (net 5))
 (segment (start 45.212 21.776081) (end 44.848999 22.139082) (width 0.25) (layer F.Cu) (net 5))
 (segment (start 45.212 20.574) (end 45.212 21.776081) (width 0.25) (layer F.Cu) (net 5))
 (segment (start 47.752 20.574) (end 49.784 18.542) (width 0.25) (layer F.Cu) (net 6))
 (segment (start 52.324 18.542) (end 55.372 15.494) (width 0.25) (layer F.Cu) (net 6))
 (segment (start 49.784 18.542) (end 52.324 18.542) (width 0.25) (layer F.Cu) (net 6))
 (segment (start 47.714001 43.904001) (end 48.514 44.704) (width 0.25) (layer F.Cu) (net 6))
 (segment (start 47.388999 43.578999) (end 47.714001 43.904001) (width 0.25) (layer F.Cu) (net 6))
 (segment (start 47.388999 22.139082) (end 47.388999 43.578999) (width 0.25) (layer F.Cu) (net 6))
 (segment (start 47.752 21.776081) (end 47.388999 22.139082) (width 0.25) (layer F.Cu) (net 6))
 (segment (start 47.752 20.574) (end 47.752 21.776081) (width 0.25) (layer F.Cu) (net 6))
 (segment (start 55.372 21.776081) (end 57.658 24.062081) (width 0.25) (layer F.Cu) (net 7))
 (segment (start 55.372 20.574) (end 55.372 21.776081) (width 0.25) (layer F.Cu) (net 7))
 (segment (start 57.658 24.062081) (end 57.658 24.13) (width 0.25) (layer F.Cu) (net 7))
 (segment (start 57.658 24.13) (end 60.706 27.178) (width 0.25) (layer F.Cu) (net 7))
 (segment (start 60.706 27.178) (end 67.056 27.178) (width 0.25) (layer F.Cu) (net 7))
 (segment (start 67.056 27.178) (end 67.818 27.94) (width 0.25) (layer F.Cu) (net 7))
 (segment (start 67.818 27.94) (end 67.818 39.37) (width 0.25) (layer F.Cu) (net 7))
 (segment (start 65.024 42.164) (end 63.754 42.164) (width 0.25) (layer F.Cu) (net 7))
 (segment (start 67.818 39.37) (end 65.024 42.164) (width 0.25) (layer F.Cu) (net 7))
 (segment (start 42.926 68.58) (end 44.704 70.358) (width 0.25) (layer F.Cu) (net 8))
 (segment (start 44.704 70.358) (end 49.53 70.358) (width 0.25) (layer F.Cu) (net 8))
 (segment (start 49.53 70.358) (end 53.086 66.802) (width 0.25) (layer F.Cu) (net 8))
 (segment (start 57.912 68.863) (end 57.912 69.088) (width 0.25) (layer F.Cu) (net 8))
 (segment (start 55.851 66.802) (end 57.912 68.863) (width 0.25) (layer F.Cu) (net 8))
 (segment (start 53.086 66.802) (end 55.851 66.802) (width 0.25) (layer F.Cu) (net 8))
 (segment (start 40.894 44.704) (end 34.036 51.562) (width 0.25) (layer B.Cu) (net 9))
 (segment (start 34.036 67.31) (end 35.306 68.58) (width 0.25) (layer B.Cu) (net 9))
 (segment (start 34.036 51.562) (end 34.036 67.31) (width 0.25) (layer B.Cu) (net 9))
 (segment (start 52.832 60.452) (end 59.332 60.452) (width 0.25) (layer F.Cu) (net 10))
 (segment (start 58.332001 59.452001) (end 59.332 60.452) (width 0.25) (layer B.Cu) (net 10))
 (segment (start 57.874001 58.994001) (end 58.332001 59.452001) (width 0.25) (layer B.Cu) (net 10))
 (segment (start 57.874001 45.503999) (end 57.874001 58.994001) (width 0.25) (layer B.Cu) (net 10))
 (segment (start 58.674 44.704) (end 57.874001 45.503999) (width 0.25) (layer B.Cu) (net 10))
 (segment (start 41.767001 49.769001) (end 42.656 50.658) (width 0.25) (layer F.Cu) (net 11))
 (segment (start 39.768999 47.770999) (end 41.767001 49.769001) (width 0.25) (layer F.Cu) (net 11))
 (segment (start 38.894001 28.338999) (end 39.768999 29.213997) (width 0.25) (layer F.Cu) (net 11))
 (segment (start 39.768999 29.213997) (end 39.768999 47.770999) (width 0.25) (layer F.Cu) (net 11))
 (segment (start 36.939001 28.338999) (end 38.894001 28.338999) (width 0.25) (layer F.Cu) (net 11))
 (segment (start 35.814 29.464) (end 36.939001 28.338999) (width 0.25) (layer F.Cu) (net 11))
 (segment (start 39.767001 49.769001) (end 40.656 50.658) (width 0.25) (layer F.Cu) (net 12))
 (segment (start 37.228999 47.230999) (end 39.767001 49.769001) (width 0.25) (layer F.Cu) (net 12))
 (segment (start 37.228999 30.589001) (end 37.228999 47.230999) (width 0.25) (layer F.Cu) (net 12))
 (segment (start 38.354 29.464) (end 37.228999 30.589001) (width 0.25) (layer F.Cu) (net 12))
 (via (at 50.546 42.164) (size 0.8) (drill 0.4) (layers F.Cu B.Cu) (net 15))
 (segment (start 39.870001 49.443999) (end 43.012001 49.443999) (width 0.25) (layer B.Cu) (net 15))
 (segment (start 43.012001 49.443999) (end 47.388999 45.067001) (width 0.25) (layer B.Cu) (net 15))
 (segment (start 38.656 50.658) (end 39.870001 49.443999) (width 0.25) (layer B.Cu) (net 15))
 (segment (start 47.388999 45.067001) (end 47.388999 44.163999) (width 0.25) (layer B.Cu) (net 15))
 (segment (start 47.388999 44.163999) (end 49.388998 42.164) (width 0.25) (layer B.Cu) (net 15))
 (segment (start 49.388998 42.164) (end 50.546 42.164) (width 0.25) (layer B.Cu) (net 15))
 (via (at 53.594 39.37) (size 0.8) (drill 0.4) (layers F.Cu B.Cu) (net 15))
 (segment (start 50.546 42.164) (end 53.34 39.37) (width 0.25) (layer F.Cu) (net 15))
 (segment (start 53.34 39.37) (end 53.594 39.37) (width 0.25) (layer F.Cu) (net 15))
 (segment (start 53.594 38.804315) (end 53.594 29.464) (width 0.25) (layer B.Cu) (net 15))
 (segment (start 53.594 39.37) (end 53.594 38.804315) (width 0.25) (layer B.Cu) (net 15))
 (segment (start 56.134 37.084) (end 59.944 37.084) (width 0.25) (layer F.Cu) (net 16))
 (segment (start 40.894 29.464) (end 38.862 27.432) (width 0.25) (layer F.Cu) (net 13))
 (segment (start 36.068 27.432) (end 34.544 28.956) (width 0.25) (layer F.Cu) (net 13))
 (segment (start 38.862 27.432) (end 36.068 27.432) (width 0.25) (layer F.Cu) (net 13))
 (segment (start 34.544 28.956) (end 34.544 51.816) (width 0.25) (layer F.Cu) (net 13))
 (segment (start 43.256001 66.057999) (end 44.156 65.158) (width 0.25) (layer F.Cu) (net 13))
 (segment (start 42.930999 66.383001) (end 43.256001 66.057999) (width 0.25) (layer F.Cu) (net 13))
 (segment (start 38.567999 66.383001) (end 42.930999 66.383001) (width 0.25) (layer F.Cu) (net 13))
 (segment (start 34.222999 62.038001) (end 38.567999 66.383001) (width 0.25) (layer F.Cu) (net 13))
 (segment (start 34.222999 52.137001) (end 34.222999 62.038001) (width 0.25) (layer F.Cu) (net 13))
 (segment (start 34.544 51.816) (end 34.222999 52.137001) (width 0.25) (layer F.Cu) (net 13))
 (segment (start 42.308999 30.589001) (end 43.434 29.464) (width 0.25) (layer F.Cu) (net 14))
 (segment (start 42.308999 45.610999) (end 42.308999 30.589001) (width 0.25) (layer F.Cu) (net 14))
 (segment (start 46.482 49.784) (end 42.308999 45.610999) (width 0.25) (layer F.Cu) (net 14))
 (segment (start 46.482 53.848) (end 46.482 49.784) (width 0.25) (layer F.Cu) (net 14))
 (segment (start 39.156 65.158) (end 39.156 61.174) (width 0.25) (layer F.Cu) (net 14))
 (segment (start 39.156 61.174) (end 46.482 53.848) (width 0.25) (layer F.Cu) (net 14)))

